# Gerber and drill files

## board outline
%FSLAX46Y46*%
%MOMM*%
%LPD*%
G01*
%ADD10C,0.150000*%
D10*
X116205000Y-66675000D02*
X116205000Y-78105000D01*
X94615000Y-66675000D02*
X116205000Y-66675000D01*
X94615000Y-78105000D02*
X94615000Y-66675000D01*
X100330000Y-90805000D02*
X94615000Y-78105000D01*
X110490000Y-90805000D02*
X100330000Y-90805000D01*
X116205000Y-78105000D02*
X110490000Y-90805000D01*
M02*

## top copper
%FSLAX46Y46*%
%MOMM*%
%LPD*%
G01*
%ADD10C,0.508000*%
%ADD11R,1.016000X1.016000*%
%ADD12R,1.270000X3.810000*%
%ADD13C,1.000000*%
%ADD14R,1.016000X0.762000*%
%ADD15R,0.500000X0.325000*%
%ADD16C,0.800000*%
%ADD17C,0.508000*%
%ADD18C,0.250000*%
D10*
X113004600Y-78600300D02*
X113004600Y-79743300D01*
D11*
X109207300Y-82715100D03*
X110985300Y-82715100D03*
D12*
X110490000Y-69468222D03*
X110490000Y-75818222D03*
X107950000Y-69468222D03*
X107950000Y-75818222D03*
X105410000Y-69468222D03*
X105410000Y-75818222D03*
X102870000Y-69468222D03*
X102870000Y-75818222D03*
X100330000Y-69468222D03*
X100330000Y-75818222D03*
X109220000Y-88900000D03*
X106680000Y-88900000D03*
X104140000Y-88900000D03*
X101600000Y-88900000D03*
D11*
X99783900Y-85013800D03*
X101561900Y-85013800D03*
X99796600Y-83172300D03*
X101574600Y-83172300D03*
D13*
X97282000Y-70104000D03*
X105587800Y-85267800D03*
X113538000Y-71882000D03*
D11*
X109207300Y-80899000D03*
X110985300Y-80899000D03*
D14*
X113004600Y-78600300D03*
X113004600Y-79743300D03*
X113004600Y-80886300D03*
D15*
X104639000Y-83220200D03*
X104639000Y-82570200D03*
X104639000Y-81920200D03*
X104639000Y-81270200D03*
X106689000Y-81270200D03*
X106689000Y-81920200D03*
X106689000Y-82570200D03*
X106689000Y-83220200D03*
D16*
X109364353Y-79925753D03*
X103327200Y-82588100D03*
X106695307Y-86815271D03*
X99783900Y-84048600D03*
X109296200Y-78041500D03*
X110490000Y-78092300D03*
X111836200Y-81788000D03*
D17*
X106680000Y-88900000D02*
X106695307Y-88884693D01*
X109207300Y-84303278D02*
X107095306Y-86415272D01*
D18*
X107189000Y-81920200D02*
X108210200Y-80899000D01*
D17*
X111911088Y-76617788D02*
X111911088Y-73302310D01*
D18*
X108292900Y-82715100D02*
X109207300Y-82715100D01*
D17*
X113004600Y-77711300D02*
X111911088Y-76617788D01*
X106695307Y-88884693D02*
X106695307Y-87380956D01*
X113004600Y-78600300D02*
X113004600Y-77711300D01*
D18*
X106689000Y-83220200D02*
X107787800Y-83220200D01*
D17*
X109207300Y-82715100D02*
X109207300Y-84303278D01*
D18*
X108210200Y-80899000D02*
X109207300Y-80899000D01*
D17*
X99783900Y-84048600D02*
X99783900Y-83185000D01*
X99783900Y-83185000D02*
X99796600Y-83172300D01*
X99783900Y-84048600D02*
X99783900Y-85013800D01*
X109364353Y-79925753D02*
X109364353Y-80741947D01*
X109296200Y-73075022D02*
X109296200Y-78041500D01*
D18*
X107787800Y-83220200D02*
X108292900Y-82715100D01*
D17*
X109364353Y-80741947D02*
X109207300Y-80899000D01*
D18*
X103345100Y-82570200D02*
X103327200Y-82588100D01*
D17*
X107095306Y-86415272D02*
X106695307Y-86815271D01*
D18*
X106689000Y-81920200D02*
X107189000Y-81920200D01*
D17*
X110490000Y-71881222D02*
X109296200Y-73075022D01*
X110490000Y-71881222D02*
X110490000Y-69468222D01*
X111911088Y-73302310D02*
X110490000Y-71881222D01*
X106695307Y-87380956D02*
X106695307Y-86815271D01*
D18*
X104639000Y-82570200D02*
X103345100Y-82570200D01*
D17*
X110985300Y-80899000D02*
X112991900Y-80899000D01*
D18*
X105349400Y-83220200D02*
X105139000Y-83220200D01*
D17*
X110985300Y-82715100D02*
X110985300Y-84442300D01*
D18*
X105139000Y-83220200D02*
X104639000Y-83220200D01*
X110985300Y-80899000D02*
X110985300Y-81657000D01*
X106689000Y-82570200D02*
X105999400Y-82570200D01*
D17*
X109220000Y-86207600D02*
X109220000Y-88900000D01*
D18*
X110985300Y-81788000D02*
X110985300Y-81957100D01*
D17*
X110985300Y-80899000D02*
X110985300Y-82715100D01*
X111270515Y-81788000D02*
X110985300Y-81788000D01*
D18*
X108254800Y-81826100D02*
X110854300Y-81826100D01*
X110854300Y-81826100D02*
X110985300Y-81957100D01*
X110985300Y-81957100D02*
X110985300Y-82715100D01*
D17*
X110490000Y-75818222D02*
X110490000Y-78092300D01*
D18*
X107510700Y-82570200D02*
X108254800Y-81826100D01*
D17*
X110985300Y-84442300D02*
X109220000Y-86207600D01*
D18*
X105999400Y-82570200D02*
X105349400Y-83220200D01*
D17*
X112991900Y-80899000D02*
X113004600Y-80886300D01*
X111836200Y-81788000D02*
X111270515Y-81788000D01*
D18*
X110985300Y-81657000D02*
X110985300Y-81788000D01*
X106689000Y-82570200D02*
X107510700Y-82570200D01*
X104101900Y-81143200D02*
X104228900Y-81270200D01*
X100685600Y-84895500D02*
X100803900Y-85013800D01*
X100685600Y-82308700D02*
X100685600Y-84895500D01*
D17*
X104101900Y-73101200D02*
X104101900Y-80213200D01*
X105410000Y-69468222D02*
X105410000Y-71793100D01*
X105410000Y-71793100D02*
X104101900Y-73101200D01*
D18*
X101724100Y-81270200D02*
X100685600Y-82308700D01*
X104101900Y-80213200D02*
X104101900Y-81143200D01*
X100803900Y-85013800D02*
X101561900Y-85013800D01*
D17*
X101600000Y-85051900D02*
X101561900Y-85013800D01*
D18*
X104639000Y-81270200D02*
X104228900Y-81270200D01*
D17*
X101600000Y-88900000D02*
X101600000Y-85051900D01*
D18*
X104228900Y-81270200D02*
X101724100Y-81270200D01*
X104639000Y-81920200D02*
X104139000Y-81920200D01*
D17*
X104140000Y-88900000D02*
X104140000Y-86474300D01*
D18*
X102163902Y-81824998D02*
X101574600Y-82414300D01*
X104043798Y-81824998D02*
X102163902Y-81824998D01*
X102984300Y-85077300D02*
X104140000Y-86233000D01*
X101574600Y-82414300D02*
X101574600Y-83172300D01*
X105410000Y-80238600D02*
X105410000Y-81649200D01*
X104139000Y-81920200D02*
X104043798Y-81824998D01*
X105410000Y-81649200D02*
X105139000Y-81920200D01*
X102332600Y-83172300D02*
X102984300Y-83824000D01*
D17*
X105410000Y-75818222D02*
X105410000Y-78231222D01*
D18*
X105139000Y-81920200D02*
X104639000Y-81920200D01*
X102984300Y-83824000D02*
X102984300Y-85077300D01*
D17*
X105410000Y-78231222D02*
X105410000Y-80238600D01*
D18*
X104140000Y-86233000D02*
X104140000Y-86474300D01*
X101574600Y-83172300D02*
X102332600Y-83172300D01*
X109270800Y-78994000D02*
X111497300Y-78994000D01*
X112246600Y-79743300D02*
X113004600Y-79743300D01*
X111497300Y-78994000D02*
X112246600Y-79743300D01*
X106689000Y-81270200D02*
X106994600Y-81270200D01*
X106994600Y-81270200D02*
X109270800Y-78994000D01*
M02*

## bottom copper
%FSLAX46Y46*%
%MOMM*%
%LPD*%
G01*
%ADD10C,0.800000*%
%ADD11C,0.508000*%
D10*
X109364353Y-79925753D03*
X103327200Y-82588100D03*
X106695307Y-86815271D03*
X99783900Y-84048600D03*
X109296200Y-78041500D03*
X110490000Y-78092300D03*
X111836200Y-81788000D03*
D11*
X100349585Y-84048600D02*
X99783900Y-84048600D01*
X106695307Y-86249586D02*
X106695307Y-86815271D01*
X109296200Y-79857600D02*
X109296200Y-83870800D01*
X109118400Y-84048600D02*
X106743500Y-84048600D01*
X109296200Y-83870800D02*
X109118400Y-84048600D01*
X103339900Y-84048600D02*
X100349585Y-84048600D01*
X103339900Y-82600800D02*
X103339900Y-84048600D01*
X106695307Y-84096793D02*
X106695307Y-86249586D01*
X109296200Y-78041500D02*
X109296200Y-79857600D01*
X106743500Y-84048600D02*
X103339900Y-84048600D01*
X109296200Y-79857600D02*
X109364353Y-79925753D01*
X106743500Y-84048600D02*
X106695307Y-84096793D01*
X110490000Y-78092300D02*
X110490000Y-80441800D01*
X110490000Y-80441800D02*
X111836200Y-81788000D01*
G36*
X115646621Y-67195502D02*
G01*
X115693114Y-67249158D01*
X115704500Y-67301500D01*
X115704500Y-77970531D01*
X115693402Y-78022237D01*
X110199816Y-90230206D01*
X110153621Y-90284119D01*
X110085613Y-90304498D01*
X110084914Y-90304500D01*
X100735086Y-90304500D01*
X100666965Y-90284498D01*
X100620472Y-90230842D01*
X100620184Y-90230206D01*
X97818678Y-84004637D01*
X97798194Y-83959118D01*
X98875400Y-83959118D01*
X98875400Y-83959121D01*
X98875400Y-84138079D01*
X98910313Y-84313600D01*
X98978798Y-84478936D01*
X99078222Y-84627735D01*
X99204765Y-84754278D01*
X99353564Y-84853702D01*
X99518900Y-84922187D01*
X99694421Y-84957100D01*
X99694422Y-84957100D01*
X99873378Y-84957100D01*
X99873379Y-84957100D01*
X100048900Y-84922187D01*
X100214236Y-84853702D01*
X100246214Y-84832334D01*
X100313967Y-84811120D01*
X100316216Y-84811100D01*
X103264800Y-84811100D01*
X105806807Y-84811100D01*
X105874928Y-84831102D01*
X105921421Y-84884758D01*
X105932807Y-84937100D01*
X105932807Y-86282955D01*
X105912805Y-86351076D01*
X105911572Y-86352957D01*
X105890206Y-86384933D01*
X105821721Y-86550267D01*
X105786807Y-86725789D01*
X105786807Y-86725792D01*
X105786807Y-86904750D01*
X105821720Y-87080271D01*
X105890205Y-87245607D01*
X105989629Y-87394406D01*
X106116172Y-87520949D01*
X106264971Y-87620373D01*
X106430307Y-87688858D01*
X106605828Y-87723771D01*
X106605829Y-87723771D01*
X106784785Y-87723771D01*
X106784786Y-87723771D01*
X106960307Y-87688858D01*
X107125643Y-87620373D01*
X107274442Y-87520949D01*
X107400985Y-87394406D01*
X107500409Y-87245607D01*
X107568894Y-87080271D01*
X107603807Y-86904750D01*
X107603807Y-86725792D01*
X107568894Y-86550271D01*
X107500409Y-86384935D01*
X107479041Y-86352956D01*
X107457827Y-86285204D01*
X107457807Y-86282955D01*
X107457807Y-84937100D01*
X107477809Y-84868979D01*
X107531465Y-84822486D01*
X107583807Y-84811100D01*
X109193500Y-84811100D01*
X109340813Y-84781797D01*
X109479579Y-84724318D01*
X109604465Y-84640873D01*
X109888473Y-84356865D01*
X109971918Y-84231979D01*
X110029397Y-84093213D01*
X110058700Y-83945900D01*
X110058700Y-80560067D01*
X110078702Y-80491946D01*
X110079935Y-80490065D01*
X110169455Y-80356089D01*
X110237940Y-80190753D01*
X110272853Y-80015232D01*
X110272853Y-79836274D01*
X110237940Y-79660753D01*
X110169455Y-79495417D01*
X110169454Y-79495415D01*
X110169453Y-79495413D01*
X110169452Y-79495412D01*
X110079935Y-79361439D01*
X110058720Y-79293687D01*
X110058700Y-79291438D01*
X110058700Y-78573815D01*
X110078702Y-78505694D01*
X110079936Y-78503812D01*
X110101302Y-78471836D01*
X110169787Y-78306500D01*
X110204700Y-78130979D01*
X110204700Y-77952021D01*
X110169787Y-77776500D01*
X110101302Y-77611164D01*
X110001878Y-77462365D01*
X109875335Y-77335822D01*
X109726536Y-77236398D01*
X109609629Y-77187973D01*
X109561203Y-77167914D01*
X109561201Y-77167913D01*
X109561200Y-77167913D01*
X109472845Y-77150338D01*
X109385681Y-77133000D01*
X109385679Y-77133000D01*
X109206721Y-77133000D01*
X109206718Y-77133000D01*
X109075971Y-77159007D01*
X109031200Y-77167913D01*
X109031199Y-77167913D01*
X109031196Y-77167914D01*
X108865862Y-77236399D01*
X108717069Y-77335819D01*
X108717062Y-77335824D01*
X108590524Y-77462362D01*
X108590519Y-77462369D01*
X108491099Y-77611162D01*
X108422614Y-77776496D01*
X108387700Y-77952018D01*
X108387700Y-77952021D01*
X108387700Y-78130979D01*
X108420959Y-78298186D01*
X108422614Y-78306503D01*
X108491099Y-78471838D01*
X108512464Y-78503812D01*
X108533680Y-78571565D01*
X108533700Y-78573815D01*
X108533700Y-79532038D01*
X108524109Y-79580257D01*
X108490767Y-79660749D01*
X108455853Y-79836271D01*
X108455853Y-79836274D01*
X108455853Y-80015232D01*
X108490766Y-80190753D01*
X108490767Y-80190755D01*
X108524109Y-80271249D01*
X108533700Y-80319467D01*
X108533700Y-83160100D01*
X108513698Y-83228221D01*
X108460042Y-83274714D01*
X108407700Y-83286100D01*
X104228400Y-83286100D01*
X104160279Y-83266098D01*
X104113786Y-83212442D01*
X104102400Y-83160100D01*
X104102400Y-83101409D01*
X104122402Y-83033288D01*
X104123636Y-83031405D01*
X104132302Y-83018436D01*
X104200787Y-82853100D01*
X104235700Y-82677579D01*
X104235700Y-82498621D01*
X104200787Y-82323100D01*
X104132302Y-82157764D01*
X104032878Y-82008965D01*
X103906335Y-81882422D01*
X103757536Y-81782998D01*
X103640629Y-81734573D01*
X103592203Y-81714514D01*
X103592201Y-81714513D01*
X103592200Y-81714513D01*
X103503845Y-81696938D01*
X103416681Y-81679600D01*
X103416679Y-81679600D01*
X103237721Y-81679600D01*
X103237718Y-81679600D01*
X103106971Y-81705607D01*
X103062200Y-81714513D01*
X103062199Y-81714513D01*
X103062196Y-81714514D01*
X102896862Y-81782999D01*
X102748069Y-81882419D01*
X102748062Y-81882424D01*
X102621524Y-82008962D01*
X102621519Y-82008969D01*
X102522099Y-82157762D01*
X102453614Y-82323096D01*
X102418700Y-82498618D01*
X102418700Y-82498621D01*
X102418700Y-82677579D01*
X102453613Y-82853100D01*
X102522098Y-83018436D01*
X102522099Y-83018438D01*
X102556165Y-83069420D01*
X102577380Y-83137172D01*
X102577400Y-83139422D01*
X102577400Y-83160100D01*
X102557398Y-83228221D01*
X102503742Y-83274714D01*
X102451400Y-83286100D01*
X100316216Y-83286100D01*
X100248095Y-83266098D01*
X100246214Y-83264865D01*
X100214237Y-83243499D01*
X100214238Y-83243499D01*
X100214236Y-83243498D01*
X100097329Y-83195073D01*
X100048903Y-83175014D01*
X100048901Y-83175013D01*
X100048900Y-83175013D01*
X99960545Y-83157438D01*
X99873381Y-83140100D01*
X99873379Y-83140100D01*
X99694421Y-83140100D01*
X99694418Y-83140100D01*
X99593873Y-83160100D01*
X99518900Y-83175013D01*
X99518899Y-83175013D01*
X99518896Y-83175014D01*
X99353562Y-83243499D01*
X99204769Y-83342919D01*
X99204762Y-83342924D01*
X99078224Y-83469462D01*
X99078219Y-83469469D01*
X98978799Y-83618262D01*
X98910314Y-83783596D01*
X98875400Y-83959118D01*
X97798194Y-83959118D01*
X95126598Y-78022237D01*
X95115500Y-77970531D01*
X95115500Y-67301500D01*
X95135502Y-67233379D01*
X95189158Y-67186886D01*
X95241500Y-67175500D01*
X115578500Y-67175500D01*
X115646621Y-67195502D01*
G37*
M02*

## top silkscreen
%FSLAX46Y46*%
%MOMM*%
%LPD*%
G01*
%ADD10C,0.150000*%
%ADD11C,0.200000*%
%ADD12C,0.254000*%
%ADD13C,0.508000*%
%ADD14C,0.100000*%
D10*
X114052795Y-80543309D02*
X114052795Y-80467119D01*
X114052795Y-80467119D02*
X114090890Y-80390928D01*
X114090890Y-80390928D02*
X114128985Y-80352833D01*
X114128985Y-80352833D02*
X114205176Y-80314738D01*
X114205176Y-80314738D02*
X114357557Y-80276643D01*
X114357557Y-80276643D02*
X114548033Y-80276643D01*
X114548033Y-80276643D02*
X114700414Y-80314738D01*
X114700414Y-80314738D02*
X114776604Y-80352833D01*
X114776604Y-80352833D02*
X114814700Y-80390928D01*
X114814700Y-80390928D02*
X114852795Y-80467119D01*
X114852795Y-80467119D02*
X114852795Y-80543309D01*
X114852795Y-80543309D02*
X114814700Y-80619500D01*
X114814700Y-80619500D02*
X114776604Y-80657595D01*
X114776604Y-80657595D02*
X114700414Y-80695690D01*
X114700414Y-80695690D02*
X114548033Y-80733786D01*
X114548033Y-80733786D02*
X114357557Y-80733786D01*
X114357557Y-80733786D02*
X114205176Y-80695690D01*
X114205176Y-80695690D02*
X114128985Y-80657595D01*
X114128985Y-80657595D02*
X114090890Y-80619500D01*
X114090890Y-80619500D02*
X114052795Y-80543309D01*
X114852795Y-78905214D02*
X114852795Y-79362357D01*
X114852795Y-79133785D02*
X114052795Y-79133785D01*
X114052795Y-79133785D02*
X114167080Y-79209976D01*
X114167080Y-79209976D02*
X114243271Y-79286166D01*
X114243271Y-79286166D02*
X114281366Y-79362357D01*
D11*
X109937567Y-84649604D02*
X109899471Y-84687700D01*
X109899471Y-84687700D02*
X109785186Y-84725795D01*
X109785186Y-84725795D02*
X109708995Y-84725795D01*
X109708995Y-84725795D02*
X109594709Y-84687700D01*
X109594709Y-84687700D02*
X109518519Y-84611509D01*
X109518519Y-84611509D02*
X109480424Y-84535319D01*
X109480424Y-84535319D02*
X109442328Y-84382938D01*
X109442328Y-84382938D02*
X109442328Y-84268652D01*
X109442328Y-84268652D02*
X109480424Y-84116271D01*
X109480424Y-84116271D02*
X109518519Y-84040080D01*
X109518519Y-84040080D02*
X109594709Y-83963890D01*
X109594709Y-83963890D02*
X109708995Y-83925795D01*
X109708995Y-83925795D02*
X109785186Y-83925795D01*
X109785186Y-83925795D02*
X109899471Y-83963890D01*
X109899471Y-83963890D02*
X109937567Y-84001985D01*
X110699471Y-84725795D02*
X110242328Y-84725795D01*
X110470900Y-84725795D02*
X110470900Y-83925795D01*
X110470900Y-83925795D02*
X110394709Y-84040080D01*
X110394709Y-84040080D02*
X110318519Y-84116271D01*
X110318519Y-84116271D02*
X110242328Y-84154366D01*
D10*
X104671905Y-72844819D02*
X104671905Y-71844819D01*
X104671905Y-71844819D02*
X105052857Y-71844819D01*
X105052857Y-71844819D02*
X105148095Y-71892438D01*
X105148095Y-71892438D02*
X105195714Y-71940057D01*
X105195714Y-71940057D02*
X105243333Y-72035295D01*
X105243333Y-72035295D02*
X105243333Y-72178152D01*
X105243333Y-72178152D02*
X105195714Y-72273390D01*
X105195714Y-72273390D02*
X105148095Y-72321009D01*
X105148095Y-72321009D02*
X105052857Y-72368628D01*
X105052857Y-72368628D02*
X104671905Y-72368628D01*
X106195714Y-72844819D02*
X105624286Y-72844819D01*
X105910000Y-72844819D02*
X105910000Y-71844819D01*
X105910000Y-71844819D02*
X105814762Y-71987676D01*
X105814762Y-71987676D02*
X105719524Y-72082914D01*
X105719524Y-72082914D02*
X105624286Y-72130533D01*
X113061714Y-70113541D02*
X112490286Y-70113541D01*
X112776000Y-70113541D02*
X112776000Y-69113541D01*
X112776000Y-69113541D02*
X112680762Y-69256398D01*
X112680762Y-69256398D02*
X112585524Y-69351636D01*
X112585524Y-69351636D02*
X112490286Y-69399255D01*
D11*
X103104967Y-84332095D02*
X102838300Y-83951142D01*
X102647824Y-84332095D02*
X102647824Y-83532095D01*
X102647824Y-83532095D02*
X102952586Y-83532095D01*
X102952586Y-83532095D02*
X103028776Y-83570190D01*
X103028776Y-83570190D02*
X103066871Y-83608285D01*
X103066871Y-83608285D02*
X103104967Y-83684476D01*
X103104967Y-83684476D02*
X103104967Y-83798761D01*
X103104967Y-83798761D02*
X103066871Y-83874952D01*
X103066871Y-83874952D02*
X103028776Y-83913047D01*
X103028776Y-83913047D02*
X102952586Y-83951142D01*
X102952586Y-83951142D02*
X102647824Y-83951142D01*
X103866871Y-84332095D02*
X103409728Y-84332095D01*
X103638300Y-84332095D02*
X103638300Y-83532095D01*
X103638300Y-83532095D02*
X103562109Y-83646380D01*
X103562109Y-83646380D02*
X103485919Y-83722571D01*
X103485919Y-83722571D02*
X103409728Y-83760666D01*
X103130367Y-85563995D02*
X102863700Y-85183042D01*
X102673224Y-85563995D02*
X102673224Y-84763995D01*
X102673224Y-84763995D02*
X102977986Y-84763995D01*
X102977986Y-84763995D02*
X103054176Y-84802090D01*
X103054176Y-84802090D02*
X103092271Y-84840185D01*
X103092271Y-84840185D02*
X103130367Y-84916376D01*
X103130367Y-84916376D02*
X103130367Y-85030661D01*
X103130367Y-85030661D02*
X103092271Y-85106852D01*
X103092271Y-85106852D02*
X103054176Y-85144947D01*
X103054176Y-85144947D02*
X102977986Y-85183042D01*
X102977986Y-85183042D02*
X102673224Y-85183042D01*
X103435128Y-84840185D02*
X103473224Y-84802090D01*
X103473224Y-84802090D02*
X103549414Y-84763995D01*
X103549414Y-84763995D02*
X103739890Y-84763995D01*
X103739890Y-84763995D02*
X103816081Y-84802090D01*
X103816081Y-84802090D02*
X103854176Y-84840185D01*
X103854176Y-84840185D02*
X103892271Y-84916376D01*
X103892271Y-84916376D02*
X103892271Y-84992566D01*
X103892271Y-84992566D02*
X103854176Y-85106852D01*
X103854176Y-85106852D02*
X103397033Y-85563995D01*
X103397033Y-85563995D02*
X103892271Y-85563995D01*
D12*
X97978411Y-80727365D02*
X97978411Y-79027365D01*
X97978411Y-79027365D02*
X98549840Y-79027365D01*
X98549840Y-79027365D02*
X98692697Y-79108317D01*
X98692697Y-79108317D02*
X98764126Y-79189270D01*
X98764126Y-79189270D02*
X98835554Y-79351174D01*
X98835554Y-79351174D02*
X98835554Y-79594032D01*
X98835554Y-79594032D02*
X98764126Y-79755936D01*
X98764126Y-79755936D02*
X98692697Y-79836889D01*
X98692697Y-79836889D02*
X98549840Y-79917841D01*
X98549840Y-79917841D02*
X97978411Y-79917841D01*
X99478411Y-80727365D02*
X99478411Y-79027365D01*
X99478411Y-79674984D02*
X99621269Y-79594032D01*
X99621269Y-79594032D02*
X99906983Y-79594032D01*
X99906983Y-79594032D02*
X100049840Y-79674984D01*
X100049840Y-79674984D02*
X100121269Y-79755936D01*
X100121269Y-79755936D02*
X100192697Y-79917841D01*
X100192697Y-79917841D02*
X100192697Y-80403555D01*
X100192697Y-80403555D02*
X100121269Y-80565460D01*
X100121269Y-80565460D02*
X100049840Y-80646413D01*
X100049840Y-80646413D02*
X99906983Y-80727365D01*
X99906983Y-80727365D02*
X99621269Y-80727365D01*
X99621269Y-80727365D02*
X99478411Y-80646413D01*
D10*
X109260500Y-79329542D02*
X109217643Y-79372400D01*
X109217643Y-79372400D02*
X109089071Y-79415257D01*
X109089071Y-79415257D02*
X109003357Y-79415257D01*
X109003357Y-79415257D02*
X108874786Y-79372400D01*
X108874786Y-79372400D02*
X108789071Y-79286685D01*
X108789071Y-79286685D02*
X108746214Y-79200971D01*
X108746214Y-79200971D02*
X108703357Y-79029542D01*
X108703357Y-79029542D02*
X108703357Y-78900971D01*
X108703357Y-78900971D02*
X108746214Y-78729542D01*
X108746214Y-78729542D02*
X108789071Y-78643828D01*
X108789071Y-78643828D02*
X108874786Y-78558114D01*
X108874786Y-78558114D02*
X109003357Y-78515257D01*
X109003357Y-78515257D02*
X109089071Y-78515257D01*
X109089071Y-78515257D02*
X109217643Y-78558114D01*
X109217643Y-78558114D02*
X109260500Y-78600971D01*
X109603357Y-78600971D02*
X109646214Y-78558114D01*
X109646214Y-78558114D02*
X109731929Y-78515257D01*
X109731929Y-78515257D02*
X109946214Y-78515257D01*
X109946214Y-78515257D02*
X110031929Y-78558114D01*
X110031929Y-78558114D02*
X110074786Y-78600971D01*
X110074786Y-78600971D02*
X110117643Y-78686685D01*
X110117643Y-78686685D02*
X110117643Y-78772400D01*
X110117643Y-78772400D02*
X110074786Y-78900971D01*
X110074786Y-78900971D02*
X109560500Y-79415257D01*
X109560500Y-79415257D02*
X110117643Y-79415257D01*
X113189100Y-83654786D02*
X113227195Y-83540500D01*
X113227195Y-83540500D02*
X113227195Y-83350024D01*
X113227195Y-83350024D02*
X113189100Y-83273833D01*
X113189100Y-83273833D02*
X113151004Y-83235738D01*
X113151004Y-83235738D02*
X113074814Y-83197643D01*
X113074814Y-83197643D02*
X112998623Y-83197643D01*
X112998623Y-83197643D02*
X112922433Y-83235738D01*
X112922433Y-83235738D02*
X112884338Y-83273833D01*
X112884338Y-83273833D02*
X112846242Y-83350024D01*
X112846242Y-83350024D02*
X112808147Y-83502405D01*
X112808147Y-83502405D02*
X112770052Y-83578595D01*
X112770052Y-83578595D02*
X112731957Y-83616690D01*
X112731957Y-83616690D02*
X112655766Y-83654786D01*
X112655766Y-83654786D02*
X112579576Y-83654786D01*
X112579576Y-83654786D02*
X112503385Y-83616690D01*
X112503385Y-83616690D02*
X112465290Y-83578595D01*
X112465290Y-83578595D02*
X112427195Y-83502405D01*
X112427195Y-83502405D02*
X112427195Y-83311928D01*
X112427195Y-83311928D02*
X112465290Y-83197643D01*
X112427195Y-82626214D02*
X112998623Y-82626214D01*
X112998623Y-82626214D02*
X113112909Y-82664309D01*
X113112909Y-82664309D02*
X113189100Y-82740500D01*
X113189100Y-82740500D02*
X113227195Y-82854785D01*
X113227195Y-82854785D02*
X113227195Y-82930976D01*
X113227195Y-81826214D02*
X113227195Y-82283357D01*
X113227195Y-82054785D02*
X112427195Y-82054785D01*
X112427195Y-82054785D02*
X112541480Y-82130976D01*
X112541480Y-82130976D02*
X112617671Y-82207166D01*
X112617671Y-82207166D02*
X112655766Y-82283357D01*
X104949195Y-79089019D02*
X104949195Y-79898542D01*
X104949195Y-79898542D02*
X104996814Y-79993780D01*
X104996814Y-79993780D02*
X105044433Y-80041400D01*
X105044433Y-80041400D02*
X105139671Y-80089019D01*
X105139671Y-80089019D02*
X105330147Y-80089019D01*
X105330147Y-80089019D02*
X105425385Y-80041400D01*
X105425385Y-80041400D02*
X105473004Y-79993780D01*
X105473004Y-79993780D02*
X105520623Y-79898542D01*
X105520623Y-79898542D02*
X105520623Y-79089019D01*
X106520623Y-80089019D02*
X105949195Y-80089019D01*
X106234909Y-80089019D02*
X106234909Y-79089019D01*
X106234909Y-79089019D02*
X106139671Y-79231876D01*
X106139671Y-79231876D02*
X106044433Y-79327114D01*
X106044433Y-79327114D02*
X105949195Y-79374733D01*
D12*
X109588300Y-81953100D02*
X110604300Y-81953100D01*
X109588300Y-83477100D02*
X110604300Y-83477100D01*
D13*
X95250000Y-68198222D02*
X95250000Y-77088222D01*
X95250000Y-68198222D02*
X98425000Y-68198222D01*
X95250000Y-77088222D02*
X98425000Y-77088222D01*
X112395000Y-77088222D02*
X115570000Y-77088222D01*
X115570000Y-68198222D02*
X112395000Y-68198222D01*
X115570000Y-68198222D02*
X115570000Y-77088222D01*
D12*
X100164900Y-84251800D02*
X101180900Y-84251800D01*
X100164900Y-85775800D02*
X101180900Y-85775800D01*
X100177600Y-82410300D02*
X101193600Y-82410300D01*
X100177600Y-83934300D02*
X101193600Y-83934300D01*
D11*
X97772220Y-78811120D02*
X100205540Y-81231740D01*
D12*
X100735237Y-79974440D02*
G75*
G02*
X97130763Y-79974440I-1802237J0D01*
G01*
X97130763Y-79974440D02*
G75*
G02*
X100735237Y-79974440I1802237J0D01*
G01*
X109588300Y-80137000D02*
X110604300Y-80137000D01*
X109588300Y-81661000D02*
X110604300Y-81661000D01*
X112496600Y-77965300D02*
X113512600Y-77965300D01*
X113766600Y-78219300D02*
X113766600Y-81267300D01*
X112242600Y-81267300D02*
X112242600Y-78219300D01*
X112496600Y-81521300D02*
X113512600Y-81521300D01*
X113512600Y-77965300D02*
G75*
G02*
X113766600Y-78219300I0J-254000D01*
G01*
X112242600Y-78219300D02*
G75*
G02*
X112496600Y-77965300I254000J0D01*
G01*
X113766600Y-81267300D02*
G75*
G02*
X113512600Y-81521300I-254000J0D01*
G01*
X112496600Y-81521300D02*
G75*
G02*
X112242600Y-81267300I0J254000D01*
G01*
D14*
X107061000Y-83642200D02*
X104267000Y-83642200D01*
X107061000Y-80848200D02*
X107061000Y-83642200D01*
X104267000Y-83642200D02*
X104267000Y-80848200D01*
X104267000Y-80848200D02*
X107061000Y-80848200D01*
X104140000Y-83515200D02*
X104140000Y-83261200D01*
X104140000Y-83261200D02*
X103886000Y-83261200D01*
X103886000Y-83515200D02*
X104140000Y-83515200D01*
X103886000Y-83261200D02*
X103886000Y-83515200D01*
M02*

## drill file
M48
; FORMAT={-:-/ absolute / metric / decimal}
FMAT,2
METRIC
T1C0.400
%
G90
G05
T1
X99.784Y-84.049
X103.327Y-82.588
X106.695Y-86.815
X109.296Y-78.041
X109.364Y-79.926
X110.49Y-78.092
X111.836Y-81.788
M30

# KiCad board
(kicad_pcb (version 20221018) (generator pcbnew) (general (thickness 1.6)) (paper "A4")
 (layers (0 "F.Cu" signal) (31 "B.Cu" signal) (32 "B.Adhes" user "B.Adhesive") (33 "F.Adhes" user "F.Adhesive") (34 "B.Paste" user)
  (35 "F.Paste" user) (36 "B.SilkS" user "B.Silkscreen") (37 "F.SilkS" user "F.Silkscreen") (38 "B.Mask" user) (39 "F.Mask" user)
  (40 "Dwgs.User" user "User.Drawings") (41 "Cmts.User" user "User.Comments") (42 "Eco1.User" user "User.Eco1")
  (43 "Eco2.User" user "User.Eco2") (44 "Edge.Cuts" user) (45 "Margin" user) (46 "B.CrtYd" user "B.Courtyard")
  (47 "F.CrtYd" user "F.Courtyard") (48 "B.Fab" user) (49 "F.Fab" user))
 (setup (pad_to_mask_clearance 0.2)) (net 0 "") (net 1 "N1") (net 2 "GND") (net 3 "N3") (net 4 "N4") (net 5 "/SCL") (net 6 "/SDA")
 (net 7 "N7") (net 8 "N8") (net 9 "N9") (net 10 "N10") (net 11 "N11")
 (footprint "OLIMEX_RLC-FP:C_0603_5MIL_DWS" (layer "F.Cu") (at 110.0963 82.7151)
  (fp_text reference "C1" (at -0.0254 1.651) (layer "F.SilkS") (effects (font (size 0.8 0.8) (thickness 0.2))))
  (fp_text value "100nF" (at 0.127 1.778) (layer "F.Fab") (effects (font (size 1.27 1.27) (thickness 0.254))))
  (fp_line (start -0.508 -0.762) (end 0.508 -0.762) (stroke (width 0.254) (type solid)) (layer "F.SilkS"))
  (fp_line (start -0.508 0.762) (end 0.508 0.762) (stroke (width 0.254) (type solid)) (layer "F.SilkS"))
  (pad "1" smd rect (at -0.889 0) (size 1.016 1.016) (layers "F.Cu" "F.Paste" "F.Mask") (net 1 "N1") (solder_mask_margin 0.0508)
   (clearance 0.0508))
  (pad "2" smd rect (at 0.889 0) (size 1.016 1.016) (layers "F.Cu" "F.Paste" "F.Mask") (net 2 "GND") (solder_mask_margin 0.0508)
   (clearance 0.0508)))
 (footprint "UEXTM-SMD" (layer "F.Cu") (at 105.41 72.643222)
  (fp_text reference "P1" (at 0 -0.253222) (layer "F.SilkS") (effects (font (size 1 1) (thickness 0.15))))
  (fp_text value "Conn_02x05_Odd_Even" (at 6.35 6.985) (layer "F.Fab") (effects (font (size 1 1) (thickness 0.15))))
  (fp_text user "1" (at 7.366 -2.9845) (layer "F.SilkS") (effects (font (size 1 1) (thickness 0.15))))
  (fp_line (start -10.16 -4.445) (end -10.16 4.445) (stroke (width 0.508) (type solid)) (layer "F.SilkS"))
  (fp_line (start -10.16 -4.445) (end -6.985 -4.445) (stroke (width 0.508) (type solid)) (layer "F.SilkS"))
  (fp_line (start -10.16 4.445) (end -6.985 4.445) (stroke (width 0.508) (type solid)) (layer "F.SilkS"))
  (fp_line (start 6.985 4.445) (end 10.16 4.445) (stroke (width 0.508) (type solid)) (layer "F.SilkS"))
  (fp_line (start 10.16 -4.445) (end 6.985 -4.445) (stroke (width 0.508) (type solid)) (layer "F.SilkS"))
  (fp_line (start 10.16 -4.445) (end 10.16 4.445) (stroke (width 0.508) (type solid)) (layer "F.SilkS"))
  (pad "1" smd rect (at 5.08 -3.175) (size 1.27 3.81) (layers "F.Cu" "F.Paste" "F.Mask") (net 1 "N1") (solder_mask_margin 0.0508)
   (solder_paste_margin 0.0508) (clearance 0.0508))
  (pad "2" smd rect (at 5.08 3.175) (size 1.27 3.81) (layers "F.Cu" "F.Paste" "F.Mask") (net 2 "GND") (solder_mask_margin 0.0508)
   (solder_paste_margin 0.0508) (clearance 0.0508))
  (pad "3" smd rect (at 2.54 -3.175) (size 1.27 3.81) (layers "F.Cu" "F.Paste" "F.Mask") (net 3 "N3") (solder_mask_margin 0.0508)
   (solder_paste_margin 0.0508) (clearance 0.0508))
  (pad "4" smd rect (at 2.54 3.175) (size 1.27 3.81) (layers "F.Cu" "F.Paste" "F.Mask") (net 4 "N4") (solder_mask_margin 0.0508)
   (solder_paste_margin 0.0508) (clearance 0.0508))
  (pad "5" smd rect (at 0 -3.175) (size 1.27 3.81) (layers "F.Cu" "F.Paste" "F.Mask") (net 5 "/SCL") (solder_mask_margin 0.0508)
   (solder_paste_margin 0.0508) (clearance 0.0508))
  (pad "6" smd rect (at 0 3.175) (size 1.27 3.81) (layers "F.Cu" "F.Paste" "F.Mask") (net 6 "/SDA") (solder_mask_margin 0.0508)
   (solder_paste_margin 0.0508) (clearance 0.0508))
  (pad "7" smd rect (at -2.54 -3.175) (size 1.27 3.81) (layers "F.Cu" "F.Paste" "F.Mask") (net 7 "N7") (solder_mask_margin 0.0508)
   (solder_paste_margin 0.0508) (clearance 0.0508))
  (pad "8" smd rect (at -2.54 3.175) (size 1.27 3.81) (layers "F.Cu" "F.Paste" "F.Mask") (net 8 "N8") (solder_mask_margin 0.0508)
   (solder_paste_margin 0.0508) (clearance 0.0508))
  (pad "9" smd rect (at -5.08 -3.175) (size 1.27 3.81) (layers "F.Cu" "F.Paste" "F.Mask") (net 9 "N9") (solder_mask_margin 0.0508)
   (solder_paste_margin 0.0508) (clearance 0.0508))
  (pad "10" smd rect (at -5.08 3.175) (size 1.27 3.81) (layers "F.Cu" "F.Paste" "F.Mask") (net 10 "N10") (solder_mask_margin 0.0508)
   (solder_paste_margin 0.0508) (clearance 0.0508)))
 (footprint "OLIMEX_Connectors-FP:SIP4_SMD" (layer "F.Cu") (at 105.41 88.9 180)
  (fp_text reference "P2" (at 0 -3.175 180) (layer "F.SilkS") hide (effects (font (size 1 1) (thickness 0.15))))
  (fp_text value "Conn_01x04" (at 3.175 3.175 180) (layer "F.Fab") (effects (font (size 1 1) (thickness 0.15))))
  (pad "1" smd rect (at -3.81 0 180) (size 1.27 3.81) (layers "F.Cu" "F.Mask") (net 2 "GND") (solder_mask_margin 0.0508)
   (solder_paste_margin -0.0508) (clearance 0.0508))
  (pad "2" smd rect (at -1.27 0 180) (size 1.27 3.81) (layers "F.Cu" "F.Mask") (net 1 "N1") (solder_mask_margin 0.0508)
   (solder_paste_margin -0.0508) (clearance 0.0508))
  (pad "3" smd rect (at 1.27 0 180) (size 1.27 3.81) (layers "F.Cu" "F.Mask") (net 6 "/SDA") (solder_mask_margin 0.0508)
   (solder_paste_margin -0.0508) (clearance 0.0508))
  (pad "4" smd rect (at 3.81 0 180) (size 1.27 3.81) (layers "F.Cu" "F.Mask") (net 5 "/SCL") (solder_mask_margin 0.0508)
   (solder_paste_margin -0.0508) (clearance 0.0508)))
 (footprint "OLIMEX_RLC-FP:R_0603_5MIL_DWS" (layer "F.Cu") (at 100.6729 85.0138)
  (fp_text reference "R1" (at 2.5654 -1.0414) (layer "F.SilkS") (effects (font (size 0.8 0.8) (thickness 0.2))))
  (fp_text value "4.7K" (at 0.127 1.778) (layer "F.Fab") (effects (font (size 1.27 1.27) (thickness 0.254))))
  (fp_line (start -0.508 -0.762) (end 0.508 -0.762) (stroke (width 0.254) (type solid)) (layer "F.SilkS"))
  (fp_line (start -0.508 0.762) (end 0.508 0.762) (stroke (width 0.254) (type solid)) (layer "F.SilkS"))
  (pad "1" smd rect (at -0.889 0) (size 1.016 1.016) (layers "F.Cu" "F.Paste" "F.Mask") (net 1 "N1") (solder_mask_margin 0.0508))
  (pad "2" smd rect (at 0.889 0) (size 1.016 1.016) (layers "F.Cu" "F.Paste" "F.Mask") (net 5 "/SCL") (solder_mask_margin 0.0508)))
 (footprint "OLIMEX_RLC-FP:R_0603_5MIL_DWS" (layer "F.Cu") (at 100.6856 83.1723)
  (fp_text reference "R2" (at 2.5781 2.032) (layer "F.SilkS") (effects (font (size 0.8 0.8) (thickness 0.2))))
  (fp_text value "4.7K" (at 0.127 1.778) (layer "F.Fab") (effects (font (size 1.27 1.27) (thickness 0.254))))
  (fp_line (start -0.508 -0.762) (end 0.508 -0.762) (stroke (width 0.254) (type solid)) (layer "F.SilkS"))
  (fp_line (start -0.508 0.762) (end 0.508 0.762) (stroke (width 0.254) (type solid)) (layer "F.SilkS"))
  (pad "1" smd rect (at -0.889 0) (size 1.016 1.016) (layers "F.Cu" "F.Paste" "F.Mask") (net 1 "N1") (solder_mask_margin 0.0508))
  (pad "2" smd rect (at 0.889 0) (size 1.016 1.016) (layers "F.Cu" "F.Paste" "F.Mask") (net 6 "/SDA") (solder_mask_margin 0.0508)))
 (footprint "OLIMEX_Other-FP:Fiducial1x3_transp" (layer "F.Cu") (at 97.282 70.104)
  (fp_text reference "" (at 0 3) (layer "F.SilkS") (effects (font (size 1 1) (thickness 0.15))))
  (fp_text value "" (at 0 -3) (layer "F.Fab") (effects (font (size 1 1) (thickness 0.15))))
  (pad "Fid1" connect circle (at 0 0) (size 1 1) (layers "F.Cu" "F.Mask") (solder_mask_margin 0.127) (clearance 1.016) (zone_connect 0)))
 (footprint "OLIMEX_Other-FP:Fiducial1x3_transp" (layer "F.Cu") (at 105.5878 85.2678)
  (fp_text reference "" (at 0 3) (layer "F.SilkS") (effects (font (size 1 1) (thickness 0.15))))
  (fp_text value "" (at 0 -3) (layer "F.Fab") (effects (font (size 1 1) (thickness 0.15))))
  (pad "Fid1" connect circle (at 0 0) (size 1 1) (layers "F.Cu" "F.Mask") (solder_mask_margin 0.127) (clearance 1.016) (zone_connect 0)))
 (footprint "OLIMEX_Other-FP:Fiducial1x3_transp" (layer "F.Cu") (at 113.538 71.882)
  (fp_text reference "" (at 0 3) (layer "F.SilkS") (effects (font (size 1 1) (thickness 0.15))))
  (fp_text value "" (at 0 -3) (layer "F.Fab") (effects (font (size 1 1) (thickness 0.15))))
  (pad "Fid1" connect circle (at 0 0) (size 1 1) (layers "F.Cu" "F.Mask") (solder_mask_margin 0.127) (clearance 1.016) (zone_connect 0)))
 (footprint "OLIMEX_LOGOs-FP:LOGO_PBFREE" (layer "F.Cu") (at 99.1362 80.2894)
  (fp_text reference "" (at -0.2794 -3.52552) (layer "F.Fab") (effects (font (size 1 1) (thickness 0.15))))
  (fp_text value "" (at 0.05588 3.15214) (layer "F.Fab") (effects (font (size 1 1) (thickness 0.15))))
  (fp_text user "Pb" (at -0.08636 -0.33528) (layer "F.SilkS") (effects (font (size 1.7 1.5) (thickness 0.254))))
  (fp_line (start -1.36398 -1.47828) (end 1.06934 0.94234) (stroke (width 0.2) (type solid)) (layer "F.SilkS"))
  (fp_circle (center -0.2032 -0.31496) (end 0.90678 -1.73482) (stroke (width 0.254) (type solid)) (fill none) (layer "F.SilkS")))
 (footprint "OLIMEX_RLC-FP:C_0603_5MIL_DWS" (layer "F.Cu") (at 110.0963 80.899)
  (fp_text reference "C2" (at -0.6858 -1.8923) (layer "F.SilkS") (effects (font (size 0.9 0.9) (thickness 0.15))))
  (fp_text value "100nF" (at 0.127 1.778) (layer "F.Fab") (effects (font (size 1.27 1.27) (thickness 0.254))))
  (fp_line (start -0.508 -0.762) (end 0.508 -0.762) (stroke (width 0.254) (type solid)) (layer "F.SilkS"))
  (fp_line (start -0.508 0.762) (end 0.508 0.762) (stroke (width 0.254) (type solid)) (layer "F.SilkS"))
  (pad "1" smd rect (at -0.889 0) (size 1.016 1.016) (layers "F.Cu" "F.Paste" "F.Mask") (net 1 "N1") (solder_mask_margin 0.0508)
   (clearance 0.0508))
  (pad "2" smd rect (at 0.889 0) (size 1.016 1.016) (layers "F.Cu" "F.Paste" "F.Mask") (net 2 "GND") (solder_mask_margin 0.0508)
   (clearance 0.0508)))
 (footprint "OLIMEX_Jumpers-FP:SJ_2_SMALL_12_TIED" (layer "F.Cu") (at 113.0046 79.7433 -90)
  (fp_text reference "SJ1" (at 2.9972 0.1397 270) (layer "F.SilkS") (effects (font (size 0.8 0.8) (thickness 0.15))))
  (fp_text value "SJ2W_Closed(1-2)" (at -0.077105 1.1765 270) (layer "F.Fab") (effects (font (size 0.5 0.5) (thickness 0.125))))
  (fp_line (start -1.143 0) (end 0 0) (stroke (width 0.508) (type solid)) (layer "F.Cu"))
  (fp_line (start -1.778 0.508) (end -1.778 -0.508) (stroke (width 0.254) (type solid)) (layer "F.SilkS"))
  (fp_line (start -1.524 -0.762) (end 1.524 -0.762) (stroke (width 0.254) (type solid)) (layer "F.SilkS"))
  (fp_line (start 1.524 0.762) (end -1.524 0.762) (stroke (width 0.254) (type solid)) (layer "F.SilkS"))
  (fp_line (start 1.778 0.508) (end 1.778 -0.508) (stroke (width 0.254) (type solid)) (layer "F.SilkS"))
  (fp_arc (start -1.778 -0.508) (mid -1.703605 -0.687605) (end -1.524 -0.762) (stroke (width 0.254) (type solid)) (layer "F.SilkS"))
  (fp_arc (start -1.524 0.762) (mid -1.703605 0.687605) (end -1.778 0.508) (stroke (width 0.254) (type solid)) (layer "F.SilkS"))
  (fp_arc (start 1.524 -0.762) (mid 1.703605 -0.687605) (end 1.778 -0.508) (stroke (width 0.254) (type solid)) (layer "F.SilkS"))
  (fp_arc (start 1.778 0.508) (mid 1.703605 0.687605) (end 1.524 0.762) (stroke (width 0.254) (type solid)) (layer "F.SilkS"))
  (pad "1" smd rect (at -1.143 0 270) (size 0.762 1.016) (layers "F.Cu" "F.Mask") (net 1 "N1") (solder_mask_margin 0.0508)
   (solder_paste_margin -0.0508) (clearance 0.0508))
  (pad "2" smd rect (at 0 0 270) (size 0.762 1.016) (layers "F.Cu" "F.Mask") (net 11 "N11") (solder_mask_margin 0.0508)
   (solder_paste_margin -0.0508) (clearance 0.0508))
  (pad "3" smd rect (at 1.143 0 270) (size 0.762 1.016) (layers "F.Cu" "F.Mask") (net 2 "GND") (solder_mask_margin 0.0508)
   (solder_paste_margin -0.0508) (clearance 0.0508)))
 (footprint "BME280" (layer "F.Cu") (at 105.664 82.2452 180)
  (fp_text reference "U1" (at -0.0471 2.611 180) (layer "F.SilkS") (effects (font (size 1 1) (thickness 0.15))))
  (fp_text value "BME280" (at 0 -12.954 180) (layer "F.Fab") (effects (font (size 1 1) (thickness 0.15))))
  (fp_line (start -1.397 -1.397) (end 1.397 -1.397) (stroke (width 0.1) (type solid)) (layer "F.SilkS"))
  (fp_line (start -1.397 1.397) (end -1.397 -1.397) (stroke (width 0.1) (type solid)) (layer "F.SilkS"))
  (fp_line (start 1.397 -1.397) (end 1.397 1.397) (stroke (width 0.1) (type solid)) (layer "F.SilkS"))
  (fp_line (start 1.397 1.397) (end -1.397 1.397) (stroke (width 0.1) (type solid)) (layer "F.SilkS"))
  (fp_line (start 1.524 -1.27) (end 1.524 -1.016) (stroke (width 0.1) (type solid)) (layer "F.SilkS"))
  (fp_line (start 1.524 -1.016) (end 1.778 -1.016) (stroke (width 0.1) (type solid)) (layer "F.SilkS"))
  (fp_line (start 1.778 -1.27) (end 1.524 -1.27) (stroke (width 0.1) (type solid)) (layer "F.SilkS"))
  (fp_line (start 1.778 -1.016) (end 1.778 -1.27) (stroke (width 0.1) (type solid)) (layer "F.SilkS"))
  (pad "1" smd rect (at 1.025 -0.975 180) (size 0.5 0.325) (layers "F.Cu" "F.Paste" "F.Mask") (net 2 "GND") (solder_mask_margin 0.05))
  (pad "2" smd rect (at 1.025 -0.325 180) (size 0.5 0.325) (layers "F.Cu" "F.Paste" "F.Mask") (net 1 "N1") (solder_mask_margin 0.05))
  (pad "3" smd rect (at 1.025 0.325 180) (size 0.5 0.325) (layers "F.Cu" "F.Paste" "F.Mask") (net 6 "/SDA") (solder_mask_margin 0.05))
  (pad "4" smd rect (at 1.025 0.975 180) (size 0.5 0.325) (layers "F.Cu" "F.Paste" "F.Mask") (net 5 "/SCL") (solder_mask_margin 0.05))
  (pad "5" smd rect (at -1.025 0.975 180) (size 0.5 0.325) (layers "F.Cu" "F.Paste" "F.Mask") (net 11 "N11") (solder_mask_margin 0.05))
  (pad "6" smd rect (at -1.025 0.325 180) (size 0.5 0.325) (layers "F.Cu" "F.Paste" "F.Mask") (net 1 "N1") (solder_mask_margin 0.05))
  (pad "7" smd rect (at -1.025 -0.325 180) (size 0.5 0.325) (layers "F.Cu" "F.Paste" "F.Mask") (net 2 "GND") (solder_mask_margin 0.05))
  (pad "8" smd rect (at -1.025 -0.975 180) (size 0.5 0.325) (layers "F.Cu" "F.Paste" "F.Mask") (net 1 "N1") (solder_mask_margin 0.05)))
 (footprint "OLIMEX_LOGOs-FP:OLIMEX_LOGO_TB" (layer "B.Cu") (at 105.41 69.85 180)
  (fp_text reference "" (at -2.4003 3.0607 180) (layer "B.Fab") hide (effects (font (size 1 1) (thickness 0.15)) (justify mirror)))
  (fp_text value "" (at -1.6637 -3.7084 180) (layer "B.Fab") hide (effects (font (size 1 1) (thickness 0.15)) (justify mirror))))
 (gr_line (start 116.205 66.675) (end 116.205 78.105) (stroke (width 0.15) (type solid)) (layer "Edge.Cuts"))
 (gr_line (start 94.615 66.675) (end 116.205 66.675) (stroke (width 0.15) (type solid)) (layer "Edge.Cuts"))
 (gr_line (start 94.615 78.105) (end 94.615 66.675) (stroke (width 0.15) (type solid)) (layer "Edge.Cuts"))
 (gr_line (start 100.33 90.805) (end 94.615 78.105) (stroke (width 0.15) (type solid)) (layer "Edge.Cuts"))
 (gr_line (start 110.49 90.805) (end 100.33 90.805) (stroke (width 0.15) (type solid)) (layer "Edge.Cuts"))
 (gr_line (start 116.205 78.105) (end 110.49 90.805) (stroke (width 0.15) (type solid)) (layer "Edge.Cuts"))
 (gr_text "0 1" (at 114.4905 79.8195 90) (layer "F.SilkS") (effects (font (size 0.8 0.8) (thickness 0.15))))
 (segment (start 106.68 88.9) (end 106.695307 88.884693) (width 0.508) (layer "F.Cu") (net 1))
 (segment (start 109.2073 84.303278) (end 107.095306 86.415272) (width 0.508) (layer "F.Cu") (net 1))
 (segment (start 107.189 81.9202) (end 108.2102 80.899) (width 0.25) (layer "F.Cu") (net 1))
 (segment (start 111.911088 76.617788) (end 111.911088 73.30231) (width 0.508) (layer "F.Cu") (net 1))
 (segment (start 108.2929 82.7151) (end 109.2073 82.7151) (width 0.25) (layer "F.Cu") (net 1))
 (segment (start 113.0046 77.7113) (end 111.911088 76.617788) (width 0.508) (layer "F.Cu") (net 1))
 (segment (start 106.695307 88.884693) (end 106.695307 87.380956) (width 0.508) (layer "F.Cu") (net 1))
 (segment (start 113.0046 78.6003) (end 113.0046 77.7113) (width 0.508) (layer "F.Cu") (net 1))
 (segment (start 106.689 83.2202) (end 107.7878 83.2202) (width 0.25) (layer "F.Cu") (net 1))
 (segment (start 109.2073 82.7151) (end 109.2073 84.303278) (width 0.508) (layer "F.Cu") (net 1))
 (segment (start 108.2102 80.899) (end 109.2073 80.899) (width 0.25) (layer "F.Cu") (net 1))
 (segment (start 99.7839 84.0486) (end 99.7839 83.185) (width 0.508) (layer "F.Cu") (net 1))
 (segment (start 99.7839 83.185) (end 99.7966 83.1723) (width 0.508) (layer "F.Cu") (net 1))
 (segment (start 99.7839 84.0486) (end 99.7839 85.0138) (width 0.508) (layer "F.Cu") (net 1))
 (segment (start 109.364353 79.925753) (end 109.364353 80.741947) (width 0.508) (layer "F.Cu") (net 1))
 (segment (start 109.2962 73.075022) (end 109.2962 78.0415) (width 0.508) (layer "F.Cu") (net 1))
 (segment (start 107.7878 83.2202) (end 108.2929 82.7151) (width 0.25) (layer "F.Cu") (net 1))
 (segment (start 109.364353 80.741947) (end 109.2073 80.899) (width 0.508) (layer "F.Cu") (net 1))
 (segment (start 103.3451 82.5702) (end 103.3272 82.5881) (width 0.25) (layer "F.Cu") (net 1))
 (segment (start 107.095306 86.415272) (end 106.695307 86.815271) (width 0.508) (layer "F.Cu") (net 1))
 (segment (start 106.689 81.9202) (end 107.189 81.9202) (width 0.25) (layer "F.Cu") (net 1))
 (segment (start 110.49 71.881222) (end 109.2962 73.075022) (width 0.508) (layer "F.Cu") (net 1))
 (segment (start 110.49 71.881222) (end 110.49 69.468222) (width 0.508) (layer "F.Cu") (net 1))
 (segment (start 111.911088 73.30231) (end 110.49 71.881222) (width 0.508) (layer "F.Cu") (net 1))
 (segment (start 106.695307 87.380956) (end 106.695307 86.815271) (width 0.508) (layer "F.Cu") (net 1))
 (segment (start 104.639 82.5702) (end 103.3451 82.5702) (width 0.25) (layer "F.Cu") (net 1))
 (via (at 109.364353 79.925753) (size 0.8) (drill 0.4) (layers "F.Cu" "B.Cu") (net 1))
 (via (at 103.3272 82.5881) (size 0.8) (drill 0.4) (layers "F.Cu" "B.Cu") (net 1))
 (via (at 106.695307 86.815271) (size 0.8) (drill 0.4) (layers "F.Cu" "B.Cu") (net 1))
 (via (at 99.7839 84.0486) (size 0.8) (drill 0.4) (layers "F.Cu" "B.Cu") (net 1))
 (via (at 109.2962 78.0415) (size 0.8) (drill 0.4) (layers "F.Cu" "B.Cu") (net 1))
 (segment (start 100.349585 84.0486) (end 99.7839 84.0486) (width 0.508) (layer "B.Cu") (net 1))
 (segment (start 106.695307 86.249586) (end 106.695307 86.815271) (width 0.508) (layer "B.Cu") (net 1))
 (segment (start 109.2962 79.8576) (end 109.2962 83.8708) (width 0.508) (layer "B.Cu") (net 1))
 (segment (start 109.1184 84.0486) (end 106.7435 84.0486) (width 0.508) (layer "B.Cu") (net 1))
 (segment (start 109.2962 83.8708) (end 109.1184 84.0486) (width 0.508) (layer "B.Cu") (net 1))
 (segment (start 103.3399 84.0486) (end 100.349585 84.0486) (width 0.508) (layer "B.Cu") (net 1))
 (segment (start 103.3399 82.6008) (end 103.3399 84.0486) (width 0.508) (layer "B.Cu") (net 1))
 (segment (start 106.695307 84.096793) (end 106.695307 86.249586) (width 0.508) (layer "B.Cu") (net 1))
 (segment (start 109.2962 78.0415) (end 109.2962 79.8576) (width 0.508) (layer "B.Cu") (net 1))
 (segment (start 106.7435 84.0486) (end 103.3399 84.0486) (width 0.508) (layer "B.Cu") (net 1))
 (segment (start 109.2962 79.8576) (end 109.364353 79.925753) (width 0.508) (layer "B.Cu") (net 1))
 (segment (start 106.7435 84.0486) (end 106.695307 84.096793) (width 0.508) (layer "B.Cu") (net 1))
 (segment (start 110.9853 80.899) (end 112.9919 80.899) (width 0.508) (layer "F.Cu") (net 2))
 (segment (start 105.3494 83.2202) (end 105.139 83.2202) (width 0.25) (layer "F.Cu") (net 2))
 (segment (start 110.9853 82.7151) (end 110.9853 84.4423) (width 0.508) (layer "F.Cu") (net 2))
 (segment (start 105.139 83.2202) (end 104.639 83.2202) (width 0.25) (layer "F.Cu") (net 2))
 (segment (start 110.9853 80.899) (end 110.9853 81.657) (width 0.25) (layer "F.Cu") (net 2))
 (segment (start 106.689 82.5702) (end 105.9994 82.5702) (width 0.25) (layer "F.Cu") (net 2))
 (segment (start 109.22 86.2076) (end 109.22 88.9) (width 0.508) (layer "F.Cu") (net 2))
 (segment (start 110.9853 81.788) (end 110.9853 81.9571) (width 0.25) (layer "F.Cu") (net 2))
 (segment (start 110.9853 80.899) (end 110.9853 82.7151) (width 0.508) (layer "F.Cu") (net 2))
 (segment (start 111.270515 81.788) (end 110.9853 81.788) (width 0.508) (layer "F.Cu") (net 2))
 (segment (start 108.2548 81.8261) (end 110.8543 81.8261) (width 0.25) (layer "F.Cu") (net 2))
 (segment (start 110.8543 81.8261) (end 110.9853 81.9571) (width 0.25) (layer "F.Cu") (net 2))
 (segment (start 110.9853 81.9571) (end 110.9853 82.7151) (width 0.25) (layer "F.Cu") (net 2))
 (segment (start 110.49 75.818222) (end 110.49 78.0923) (width 0.508) (layer "F.Cu") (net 2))
 (segment (start 107.5107 82.5702) (end 108.2548 81.8261) (width 0.25) (layer "F.Cu") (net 2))
 (segment (start 110.9853 84.4423) (end 109.22 86.2076) (width 0.508) (layer "F.Cu") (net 2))
 (segment (start 105.9994 82.5702) (end 105.3494 83.2202) (width 0.25) (layer "F.Cu") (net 2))
 (segment (start 112.9919 80.899) (end 113.0046 80.8863) (width 0.508) (layer "F.Cu") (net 2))
 (segment (start 111.8362 81.788) (end 111.270515 81.788) (width 0.508) (layer "F.Cu") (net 2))
 (segment (start 110.9853 81.657) (end 110.9853 81.788) (width 0.25) (layer "F.Cu") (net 2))
 (segment (start 106.689 82.5702) (end 107.5107 82.5702) (width 0.25) (layer "F.Cu") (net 2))
 (via (at 110.49 78.0923) (size 0.8) (drill 0.4) (layers "F.Cu" "B.Cu") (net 2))
 (via (at 111.8362 81.788) (size 0.8) (drill 0.4) (layers "F.Cu" "B.Cu") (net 2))
 (segment (start 110.49 78.0923) (end 110.49 80.4418) (width 0.508) (layer "B.Cu") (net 2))
 (segment (start 110.49 80.4418) (end 111.8362 81.788) (width 0.508) (layer "B.Cu") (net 2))
 (segment (start 104.1019 81.1432) (end 104.2289 81.2702) (width 0.25) (layer "F.Cu") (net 5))
 (segment (start 100.6856 84.8955) (end 100.8039 85.0138) (width 0.25) (layer "F.Cu") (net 5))
 (segment (start 100.6856 82.3087) (end 100.6856 84.8955) (width 0.25) (layer "F.Cu") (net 5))
 (segment (start 104.1019 73.1012) (end 104.1019 80.2132) (width 0.508) (layer "F.Cu") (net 5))
 (segment (start 105.41 69.468222) (end 105.41 71.7931) (width 0.508) (layer "F.Cu") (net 5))
 (segment (start 105.41 71.7931) (end 104.1019 73.1012) (width 0.508) (layer "F.Cu") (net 5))
 (segment (start 101.7241 81.2702) (end 100.6856 82.3087) (width 0.25) (layer "F.Cu") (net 5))
 (segment (start 104.1019 80.2132) (end 104.1019 81.1432) (width 0.25) (layer "F.Cu") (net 5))
 (segment (start 100.8039 85.0138) (end 101.5619 85.0138) (width 0.25) (layer "F.Cu") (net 5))
 (segment (start 101.6 85.0519) (end 101.5619 85.0138) (width 0.508) (layer "F.Cu") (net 5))
 (segment (start 104.639 81.2702) (end 104.2289 81.2702) (width 0.25) (layer "F.Cu") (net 5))
 (segment (start 101.6 88.9) (end 101.6 85.0519) (width 0.508) (layer "F.Cu") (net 5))
 (segment (start 104.2289 81.2702) (end 101.7241 81.2702) (width 0.25) (layer "F.Cu") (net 5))
 (segment (start 104.639 81.9202) (end 104.139 81.9202) (width 0.25) (layer "F.Cu") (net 6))
 (segment (start 104.14 88.9) (end 104.14 86.4743) (width 0.508) (layer "F.Cu") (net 6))
 (segment (start 102.163902 81.824998) (end 101.5746 82.4143) (width 0.25) (layer "F.Cu") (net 6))
 (segment (start 104.043798 81.824998) (end 102.163902 81.824998) (width 0.25) (layer "F.Cu") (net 6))
 (segment (start 102.9843 85.0773) (end 104.14 86.233) (width 0.25) (layer "F.Cu") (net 6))
 (segment (start 101.5746 82.4143) (end 101.5746 83.1723) (width 0.25) (layer "F.Cu") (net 6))
 (segment (start 105.41 80.2386) (end 105.41 81.6492) (width 0.25) (layer "F.Cu") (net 6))
 (segment (start 104.139 81.9202) (end 104.043798 81.824998) (width 0.25) (layer "F.Cu") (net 6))
 (segment (start 105.41 81.6492) (end 105.139 81.9202) (width 0.25) (layer "F.Cu") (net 6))
 (segment (start 102.3326 83.1723) (end 102.9843 83.824) (width 0.25) (layer "F.Cu") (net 6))
 (segment (start 105.41 75.818222) (end 105.41 78.231222) (width 0.508) (layer "F.Cu") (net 6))
 (segment (start 105.139 81.9202) (end 104.639 81.9202) (width 0.25) (layer "F.Cu") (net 6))
 (segment (start 102.9843 83.824) (end 102.9843 85.0773) (width 0.25) (layer "F.Cu") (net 6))
 (segment (start 105.41 78.231222) (end 105.41 80.2386) (width 0.508) (layer "F.Cu") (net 6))
 (segment (start 104.14 86.233) (end 104.14 86.4743) (width 0.25) (layer "F.Cu") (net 6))
 (segment (start 101.5746 83.1723) (end 102.3326 83.1723) (width 0.25) (layer "F.Cu") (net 6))
 (segment (start 109.2708 78.994) (end 111.4973 78.994) (width 0.25) (layer "F.Cu") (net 11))
 (segment (start 112.2466 79.7433) (end 113.0046 79.7433) (width 0.25) (layer "F.Cu") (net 11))
 (segment (start 111.4973 78.994) (end 112.2466 79.7433) (width 0.25) (layer "F.Cu") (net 11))
 (segment (start 106.689 81.2702) (end 106.9946 81.2702) (width 0.25) (layer "F.Cu") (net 11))
 (segment (start 106.9946 81.2702) (end 109.2708 78.994) (width 0.25) (layer "F.Cu") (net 11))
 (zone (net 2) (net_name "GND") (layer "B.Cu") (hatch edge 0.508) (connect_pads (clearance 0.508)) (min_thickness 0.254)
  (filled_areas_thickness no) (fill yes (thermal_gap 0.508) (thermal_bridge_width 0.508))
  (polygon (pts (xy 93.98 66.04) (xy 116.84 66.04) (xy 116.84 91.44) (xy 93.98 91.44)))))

